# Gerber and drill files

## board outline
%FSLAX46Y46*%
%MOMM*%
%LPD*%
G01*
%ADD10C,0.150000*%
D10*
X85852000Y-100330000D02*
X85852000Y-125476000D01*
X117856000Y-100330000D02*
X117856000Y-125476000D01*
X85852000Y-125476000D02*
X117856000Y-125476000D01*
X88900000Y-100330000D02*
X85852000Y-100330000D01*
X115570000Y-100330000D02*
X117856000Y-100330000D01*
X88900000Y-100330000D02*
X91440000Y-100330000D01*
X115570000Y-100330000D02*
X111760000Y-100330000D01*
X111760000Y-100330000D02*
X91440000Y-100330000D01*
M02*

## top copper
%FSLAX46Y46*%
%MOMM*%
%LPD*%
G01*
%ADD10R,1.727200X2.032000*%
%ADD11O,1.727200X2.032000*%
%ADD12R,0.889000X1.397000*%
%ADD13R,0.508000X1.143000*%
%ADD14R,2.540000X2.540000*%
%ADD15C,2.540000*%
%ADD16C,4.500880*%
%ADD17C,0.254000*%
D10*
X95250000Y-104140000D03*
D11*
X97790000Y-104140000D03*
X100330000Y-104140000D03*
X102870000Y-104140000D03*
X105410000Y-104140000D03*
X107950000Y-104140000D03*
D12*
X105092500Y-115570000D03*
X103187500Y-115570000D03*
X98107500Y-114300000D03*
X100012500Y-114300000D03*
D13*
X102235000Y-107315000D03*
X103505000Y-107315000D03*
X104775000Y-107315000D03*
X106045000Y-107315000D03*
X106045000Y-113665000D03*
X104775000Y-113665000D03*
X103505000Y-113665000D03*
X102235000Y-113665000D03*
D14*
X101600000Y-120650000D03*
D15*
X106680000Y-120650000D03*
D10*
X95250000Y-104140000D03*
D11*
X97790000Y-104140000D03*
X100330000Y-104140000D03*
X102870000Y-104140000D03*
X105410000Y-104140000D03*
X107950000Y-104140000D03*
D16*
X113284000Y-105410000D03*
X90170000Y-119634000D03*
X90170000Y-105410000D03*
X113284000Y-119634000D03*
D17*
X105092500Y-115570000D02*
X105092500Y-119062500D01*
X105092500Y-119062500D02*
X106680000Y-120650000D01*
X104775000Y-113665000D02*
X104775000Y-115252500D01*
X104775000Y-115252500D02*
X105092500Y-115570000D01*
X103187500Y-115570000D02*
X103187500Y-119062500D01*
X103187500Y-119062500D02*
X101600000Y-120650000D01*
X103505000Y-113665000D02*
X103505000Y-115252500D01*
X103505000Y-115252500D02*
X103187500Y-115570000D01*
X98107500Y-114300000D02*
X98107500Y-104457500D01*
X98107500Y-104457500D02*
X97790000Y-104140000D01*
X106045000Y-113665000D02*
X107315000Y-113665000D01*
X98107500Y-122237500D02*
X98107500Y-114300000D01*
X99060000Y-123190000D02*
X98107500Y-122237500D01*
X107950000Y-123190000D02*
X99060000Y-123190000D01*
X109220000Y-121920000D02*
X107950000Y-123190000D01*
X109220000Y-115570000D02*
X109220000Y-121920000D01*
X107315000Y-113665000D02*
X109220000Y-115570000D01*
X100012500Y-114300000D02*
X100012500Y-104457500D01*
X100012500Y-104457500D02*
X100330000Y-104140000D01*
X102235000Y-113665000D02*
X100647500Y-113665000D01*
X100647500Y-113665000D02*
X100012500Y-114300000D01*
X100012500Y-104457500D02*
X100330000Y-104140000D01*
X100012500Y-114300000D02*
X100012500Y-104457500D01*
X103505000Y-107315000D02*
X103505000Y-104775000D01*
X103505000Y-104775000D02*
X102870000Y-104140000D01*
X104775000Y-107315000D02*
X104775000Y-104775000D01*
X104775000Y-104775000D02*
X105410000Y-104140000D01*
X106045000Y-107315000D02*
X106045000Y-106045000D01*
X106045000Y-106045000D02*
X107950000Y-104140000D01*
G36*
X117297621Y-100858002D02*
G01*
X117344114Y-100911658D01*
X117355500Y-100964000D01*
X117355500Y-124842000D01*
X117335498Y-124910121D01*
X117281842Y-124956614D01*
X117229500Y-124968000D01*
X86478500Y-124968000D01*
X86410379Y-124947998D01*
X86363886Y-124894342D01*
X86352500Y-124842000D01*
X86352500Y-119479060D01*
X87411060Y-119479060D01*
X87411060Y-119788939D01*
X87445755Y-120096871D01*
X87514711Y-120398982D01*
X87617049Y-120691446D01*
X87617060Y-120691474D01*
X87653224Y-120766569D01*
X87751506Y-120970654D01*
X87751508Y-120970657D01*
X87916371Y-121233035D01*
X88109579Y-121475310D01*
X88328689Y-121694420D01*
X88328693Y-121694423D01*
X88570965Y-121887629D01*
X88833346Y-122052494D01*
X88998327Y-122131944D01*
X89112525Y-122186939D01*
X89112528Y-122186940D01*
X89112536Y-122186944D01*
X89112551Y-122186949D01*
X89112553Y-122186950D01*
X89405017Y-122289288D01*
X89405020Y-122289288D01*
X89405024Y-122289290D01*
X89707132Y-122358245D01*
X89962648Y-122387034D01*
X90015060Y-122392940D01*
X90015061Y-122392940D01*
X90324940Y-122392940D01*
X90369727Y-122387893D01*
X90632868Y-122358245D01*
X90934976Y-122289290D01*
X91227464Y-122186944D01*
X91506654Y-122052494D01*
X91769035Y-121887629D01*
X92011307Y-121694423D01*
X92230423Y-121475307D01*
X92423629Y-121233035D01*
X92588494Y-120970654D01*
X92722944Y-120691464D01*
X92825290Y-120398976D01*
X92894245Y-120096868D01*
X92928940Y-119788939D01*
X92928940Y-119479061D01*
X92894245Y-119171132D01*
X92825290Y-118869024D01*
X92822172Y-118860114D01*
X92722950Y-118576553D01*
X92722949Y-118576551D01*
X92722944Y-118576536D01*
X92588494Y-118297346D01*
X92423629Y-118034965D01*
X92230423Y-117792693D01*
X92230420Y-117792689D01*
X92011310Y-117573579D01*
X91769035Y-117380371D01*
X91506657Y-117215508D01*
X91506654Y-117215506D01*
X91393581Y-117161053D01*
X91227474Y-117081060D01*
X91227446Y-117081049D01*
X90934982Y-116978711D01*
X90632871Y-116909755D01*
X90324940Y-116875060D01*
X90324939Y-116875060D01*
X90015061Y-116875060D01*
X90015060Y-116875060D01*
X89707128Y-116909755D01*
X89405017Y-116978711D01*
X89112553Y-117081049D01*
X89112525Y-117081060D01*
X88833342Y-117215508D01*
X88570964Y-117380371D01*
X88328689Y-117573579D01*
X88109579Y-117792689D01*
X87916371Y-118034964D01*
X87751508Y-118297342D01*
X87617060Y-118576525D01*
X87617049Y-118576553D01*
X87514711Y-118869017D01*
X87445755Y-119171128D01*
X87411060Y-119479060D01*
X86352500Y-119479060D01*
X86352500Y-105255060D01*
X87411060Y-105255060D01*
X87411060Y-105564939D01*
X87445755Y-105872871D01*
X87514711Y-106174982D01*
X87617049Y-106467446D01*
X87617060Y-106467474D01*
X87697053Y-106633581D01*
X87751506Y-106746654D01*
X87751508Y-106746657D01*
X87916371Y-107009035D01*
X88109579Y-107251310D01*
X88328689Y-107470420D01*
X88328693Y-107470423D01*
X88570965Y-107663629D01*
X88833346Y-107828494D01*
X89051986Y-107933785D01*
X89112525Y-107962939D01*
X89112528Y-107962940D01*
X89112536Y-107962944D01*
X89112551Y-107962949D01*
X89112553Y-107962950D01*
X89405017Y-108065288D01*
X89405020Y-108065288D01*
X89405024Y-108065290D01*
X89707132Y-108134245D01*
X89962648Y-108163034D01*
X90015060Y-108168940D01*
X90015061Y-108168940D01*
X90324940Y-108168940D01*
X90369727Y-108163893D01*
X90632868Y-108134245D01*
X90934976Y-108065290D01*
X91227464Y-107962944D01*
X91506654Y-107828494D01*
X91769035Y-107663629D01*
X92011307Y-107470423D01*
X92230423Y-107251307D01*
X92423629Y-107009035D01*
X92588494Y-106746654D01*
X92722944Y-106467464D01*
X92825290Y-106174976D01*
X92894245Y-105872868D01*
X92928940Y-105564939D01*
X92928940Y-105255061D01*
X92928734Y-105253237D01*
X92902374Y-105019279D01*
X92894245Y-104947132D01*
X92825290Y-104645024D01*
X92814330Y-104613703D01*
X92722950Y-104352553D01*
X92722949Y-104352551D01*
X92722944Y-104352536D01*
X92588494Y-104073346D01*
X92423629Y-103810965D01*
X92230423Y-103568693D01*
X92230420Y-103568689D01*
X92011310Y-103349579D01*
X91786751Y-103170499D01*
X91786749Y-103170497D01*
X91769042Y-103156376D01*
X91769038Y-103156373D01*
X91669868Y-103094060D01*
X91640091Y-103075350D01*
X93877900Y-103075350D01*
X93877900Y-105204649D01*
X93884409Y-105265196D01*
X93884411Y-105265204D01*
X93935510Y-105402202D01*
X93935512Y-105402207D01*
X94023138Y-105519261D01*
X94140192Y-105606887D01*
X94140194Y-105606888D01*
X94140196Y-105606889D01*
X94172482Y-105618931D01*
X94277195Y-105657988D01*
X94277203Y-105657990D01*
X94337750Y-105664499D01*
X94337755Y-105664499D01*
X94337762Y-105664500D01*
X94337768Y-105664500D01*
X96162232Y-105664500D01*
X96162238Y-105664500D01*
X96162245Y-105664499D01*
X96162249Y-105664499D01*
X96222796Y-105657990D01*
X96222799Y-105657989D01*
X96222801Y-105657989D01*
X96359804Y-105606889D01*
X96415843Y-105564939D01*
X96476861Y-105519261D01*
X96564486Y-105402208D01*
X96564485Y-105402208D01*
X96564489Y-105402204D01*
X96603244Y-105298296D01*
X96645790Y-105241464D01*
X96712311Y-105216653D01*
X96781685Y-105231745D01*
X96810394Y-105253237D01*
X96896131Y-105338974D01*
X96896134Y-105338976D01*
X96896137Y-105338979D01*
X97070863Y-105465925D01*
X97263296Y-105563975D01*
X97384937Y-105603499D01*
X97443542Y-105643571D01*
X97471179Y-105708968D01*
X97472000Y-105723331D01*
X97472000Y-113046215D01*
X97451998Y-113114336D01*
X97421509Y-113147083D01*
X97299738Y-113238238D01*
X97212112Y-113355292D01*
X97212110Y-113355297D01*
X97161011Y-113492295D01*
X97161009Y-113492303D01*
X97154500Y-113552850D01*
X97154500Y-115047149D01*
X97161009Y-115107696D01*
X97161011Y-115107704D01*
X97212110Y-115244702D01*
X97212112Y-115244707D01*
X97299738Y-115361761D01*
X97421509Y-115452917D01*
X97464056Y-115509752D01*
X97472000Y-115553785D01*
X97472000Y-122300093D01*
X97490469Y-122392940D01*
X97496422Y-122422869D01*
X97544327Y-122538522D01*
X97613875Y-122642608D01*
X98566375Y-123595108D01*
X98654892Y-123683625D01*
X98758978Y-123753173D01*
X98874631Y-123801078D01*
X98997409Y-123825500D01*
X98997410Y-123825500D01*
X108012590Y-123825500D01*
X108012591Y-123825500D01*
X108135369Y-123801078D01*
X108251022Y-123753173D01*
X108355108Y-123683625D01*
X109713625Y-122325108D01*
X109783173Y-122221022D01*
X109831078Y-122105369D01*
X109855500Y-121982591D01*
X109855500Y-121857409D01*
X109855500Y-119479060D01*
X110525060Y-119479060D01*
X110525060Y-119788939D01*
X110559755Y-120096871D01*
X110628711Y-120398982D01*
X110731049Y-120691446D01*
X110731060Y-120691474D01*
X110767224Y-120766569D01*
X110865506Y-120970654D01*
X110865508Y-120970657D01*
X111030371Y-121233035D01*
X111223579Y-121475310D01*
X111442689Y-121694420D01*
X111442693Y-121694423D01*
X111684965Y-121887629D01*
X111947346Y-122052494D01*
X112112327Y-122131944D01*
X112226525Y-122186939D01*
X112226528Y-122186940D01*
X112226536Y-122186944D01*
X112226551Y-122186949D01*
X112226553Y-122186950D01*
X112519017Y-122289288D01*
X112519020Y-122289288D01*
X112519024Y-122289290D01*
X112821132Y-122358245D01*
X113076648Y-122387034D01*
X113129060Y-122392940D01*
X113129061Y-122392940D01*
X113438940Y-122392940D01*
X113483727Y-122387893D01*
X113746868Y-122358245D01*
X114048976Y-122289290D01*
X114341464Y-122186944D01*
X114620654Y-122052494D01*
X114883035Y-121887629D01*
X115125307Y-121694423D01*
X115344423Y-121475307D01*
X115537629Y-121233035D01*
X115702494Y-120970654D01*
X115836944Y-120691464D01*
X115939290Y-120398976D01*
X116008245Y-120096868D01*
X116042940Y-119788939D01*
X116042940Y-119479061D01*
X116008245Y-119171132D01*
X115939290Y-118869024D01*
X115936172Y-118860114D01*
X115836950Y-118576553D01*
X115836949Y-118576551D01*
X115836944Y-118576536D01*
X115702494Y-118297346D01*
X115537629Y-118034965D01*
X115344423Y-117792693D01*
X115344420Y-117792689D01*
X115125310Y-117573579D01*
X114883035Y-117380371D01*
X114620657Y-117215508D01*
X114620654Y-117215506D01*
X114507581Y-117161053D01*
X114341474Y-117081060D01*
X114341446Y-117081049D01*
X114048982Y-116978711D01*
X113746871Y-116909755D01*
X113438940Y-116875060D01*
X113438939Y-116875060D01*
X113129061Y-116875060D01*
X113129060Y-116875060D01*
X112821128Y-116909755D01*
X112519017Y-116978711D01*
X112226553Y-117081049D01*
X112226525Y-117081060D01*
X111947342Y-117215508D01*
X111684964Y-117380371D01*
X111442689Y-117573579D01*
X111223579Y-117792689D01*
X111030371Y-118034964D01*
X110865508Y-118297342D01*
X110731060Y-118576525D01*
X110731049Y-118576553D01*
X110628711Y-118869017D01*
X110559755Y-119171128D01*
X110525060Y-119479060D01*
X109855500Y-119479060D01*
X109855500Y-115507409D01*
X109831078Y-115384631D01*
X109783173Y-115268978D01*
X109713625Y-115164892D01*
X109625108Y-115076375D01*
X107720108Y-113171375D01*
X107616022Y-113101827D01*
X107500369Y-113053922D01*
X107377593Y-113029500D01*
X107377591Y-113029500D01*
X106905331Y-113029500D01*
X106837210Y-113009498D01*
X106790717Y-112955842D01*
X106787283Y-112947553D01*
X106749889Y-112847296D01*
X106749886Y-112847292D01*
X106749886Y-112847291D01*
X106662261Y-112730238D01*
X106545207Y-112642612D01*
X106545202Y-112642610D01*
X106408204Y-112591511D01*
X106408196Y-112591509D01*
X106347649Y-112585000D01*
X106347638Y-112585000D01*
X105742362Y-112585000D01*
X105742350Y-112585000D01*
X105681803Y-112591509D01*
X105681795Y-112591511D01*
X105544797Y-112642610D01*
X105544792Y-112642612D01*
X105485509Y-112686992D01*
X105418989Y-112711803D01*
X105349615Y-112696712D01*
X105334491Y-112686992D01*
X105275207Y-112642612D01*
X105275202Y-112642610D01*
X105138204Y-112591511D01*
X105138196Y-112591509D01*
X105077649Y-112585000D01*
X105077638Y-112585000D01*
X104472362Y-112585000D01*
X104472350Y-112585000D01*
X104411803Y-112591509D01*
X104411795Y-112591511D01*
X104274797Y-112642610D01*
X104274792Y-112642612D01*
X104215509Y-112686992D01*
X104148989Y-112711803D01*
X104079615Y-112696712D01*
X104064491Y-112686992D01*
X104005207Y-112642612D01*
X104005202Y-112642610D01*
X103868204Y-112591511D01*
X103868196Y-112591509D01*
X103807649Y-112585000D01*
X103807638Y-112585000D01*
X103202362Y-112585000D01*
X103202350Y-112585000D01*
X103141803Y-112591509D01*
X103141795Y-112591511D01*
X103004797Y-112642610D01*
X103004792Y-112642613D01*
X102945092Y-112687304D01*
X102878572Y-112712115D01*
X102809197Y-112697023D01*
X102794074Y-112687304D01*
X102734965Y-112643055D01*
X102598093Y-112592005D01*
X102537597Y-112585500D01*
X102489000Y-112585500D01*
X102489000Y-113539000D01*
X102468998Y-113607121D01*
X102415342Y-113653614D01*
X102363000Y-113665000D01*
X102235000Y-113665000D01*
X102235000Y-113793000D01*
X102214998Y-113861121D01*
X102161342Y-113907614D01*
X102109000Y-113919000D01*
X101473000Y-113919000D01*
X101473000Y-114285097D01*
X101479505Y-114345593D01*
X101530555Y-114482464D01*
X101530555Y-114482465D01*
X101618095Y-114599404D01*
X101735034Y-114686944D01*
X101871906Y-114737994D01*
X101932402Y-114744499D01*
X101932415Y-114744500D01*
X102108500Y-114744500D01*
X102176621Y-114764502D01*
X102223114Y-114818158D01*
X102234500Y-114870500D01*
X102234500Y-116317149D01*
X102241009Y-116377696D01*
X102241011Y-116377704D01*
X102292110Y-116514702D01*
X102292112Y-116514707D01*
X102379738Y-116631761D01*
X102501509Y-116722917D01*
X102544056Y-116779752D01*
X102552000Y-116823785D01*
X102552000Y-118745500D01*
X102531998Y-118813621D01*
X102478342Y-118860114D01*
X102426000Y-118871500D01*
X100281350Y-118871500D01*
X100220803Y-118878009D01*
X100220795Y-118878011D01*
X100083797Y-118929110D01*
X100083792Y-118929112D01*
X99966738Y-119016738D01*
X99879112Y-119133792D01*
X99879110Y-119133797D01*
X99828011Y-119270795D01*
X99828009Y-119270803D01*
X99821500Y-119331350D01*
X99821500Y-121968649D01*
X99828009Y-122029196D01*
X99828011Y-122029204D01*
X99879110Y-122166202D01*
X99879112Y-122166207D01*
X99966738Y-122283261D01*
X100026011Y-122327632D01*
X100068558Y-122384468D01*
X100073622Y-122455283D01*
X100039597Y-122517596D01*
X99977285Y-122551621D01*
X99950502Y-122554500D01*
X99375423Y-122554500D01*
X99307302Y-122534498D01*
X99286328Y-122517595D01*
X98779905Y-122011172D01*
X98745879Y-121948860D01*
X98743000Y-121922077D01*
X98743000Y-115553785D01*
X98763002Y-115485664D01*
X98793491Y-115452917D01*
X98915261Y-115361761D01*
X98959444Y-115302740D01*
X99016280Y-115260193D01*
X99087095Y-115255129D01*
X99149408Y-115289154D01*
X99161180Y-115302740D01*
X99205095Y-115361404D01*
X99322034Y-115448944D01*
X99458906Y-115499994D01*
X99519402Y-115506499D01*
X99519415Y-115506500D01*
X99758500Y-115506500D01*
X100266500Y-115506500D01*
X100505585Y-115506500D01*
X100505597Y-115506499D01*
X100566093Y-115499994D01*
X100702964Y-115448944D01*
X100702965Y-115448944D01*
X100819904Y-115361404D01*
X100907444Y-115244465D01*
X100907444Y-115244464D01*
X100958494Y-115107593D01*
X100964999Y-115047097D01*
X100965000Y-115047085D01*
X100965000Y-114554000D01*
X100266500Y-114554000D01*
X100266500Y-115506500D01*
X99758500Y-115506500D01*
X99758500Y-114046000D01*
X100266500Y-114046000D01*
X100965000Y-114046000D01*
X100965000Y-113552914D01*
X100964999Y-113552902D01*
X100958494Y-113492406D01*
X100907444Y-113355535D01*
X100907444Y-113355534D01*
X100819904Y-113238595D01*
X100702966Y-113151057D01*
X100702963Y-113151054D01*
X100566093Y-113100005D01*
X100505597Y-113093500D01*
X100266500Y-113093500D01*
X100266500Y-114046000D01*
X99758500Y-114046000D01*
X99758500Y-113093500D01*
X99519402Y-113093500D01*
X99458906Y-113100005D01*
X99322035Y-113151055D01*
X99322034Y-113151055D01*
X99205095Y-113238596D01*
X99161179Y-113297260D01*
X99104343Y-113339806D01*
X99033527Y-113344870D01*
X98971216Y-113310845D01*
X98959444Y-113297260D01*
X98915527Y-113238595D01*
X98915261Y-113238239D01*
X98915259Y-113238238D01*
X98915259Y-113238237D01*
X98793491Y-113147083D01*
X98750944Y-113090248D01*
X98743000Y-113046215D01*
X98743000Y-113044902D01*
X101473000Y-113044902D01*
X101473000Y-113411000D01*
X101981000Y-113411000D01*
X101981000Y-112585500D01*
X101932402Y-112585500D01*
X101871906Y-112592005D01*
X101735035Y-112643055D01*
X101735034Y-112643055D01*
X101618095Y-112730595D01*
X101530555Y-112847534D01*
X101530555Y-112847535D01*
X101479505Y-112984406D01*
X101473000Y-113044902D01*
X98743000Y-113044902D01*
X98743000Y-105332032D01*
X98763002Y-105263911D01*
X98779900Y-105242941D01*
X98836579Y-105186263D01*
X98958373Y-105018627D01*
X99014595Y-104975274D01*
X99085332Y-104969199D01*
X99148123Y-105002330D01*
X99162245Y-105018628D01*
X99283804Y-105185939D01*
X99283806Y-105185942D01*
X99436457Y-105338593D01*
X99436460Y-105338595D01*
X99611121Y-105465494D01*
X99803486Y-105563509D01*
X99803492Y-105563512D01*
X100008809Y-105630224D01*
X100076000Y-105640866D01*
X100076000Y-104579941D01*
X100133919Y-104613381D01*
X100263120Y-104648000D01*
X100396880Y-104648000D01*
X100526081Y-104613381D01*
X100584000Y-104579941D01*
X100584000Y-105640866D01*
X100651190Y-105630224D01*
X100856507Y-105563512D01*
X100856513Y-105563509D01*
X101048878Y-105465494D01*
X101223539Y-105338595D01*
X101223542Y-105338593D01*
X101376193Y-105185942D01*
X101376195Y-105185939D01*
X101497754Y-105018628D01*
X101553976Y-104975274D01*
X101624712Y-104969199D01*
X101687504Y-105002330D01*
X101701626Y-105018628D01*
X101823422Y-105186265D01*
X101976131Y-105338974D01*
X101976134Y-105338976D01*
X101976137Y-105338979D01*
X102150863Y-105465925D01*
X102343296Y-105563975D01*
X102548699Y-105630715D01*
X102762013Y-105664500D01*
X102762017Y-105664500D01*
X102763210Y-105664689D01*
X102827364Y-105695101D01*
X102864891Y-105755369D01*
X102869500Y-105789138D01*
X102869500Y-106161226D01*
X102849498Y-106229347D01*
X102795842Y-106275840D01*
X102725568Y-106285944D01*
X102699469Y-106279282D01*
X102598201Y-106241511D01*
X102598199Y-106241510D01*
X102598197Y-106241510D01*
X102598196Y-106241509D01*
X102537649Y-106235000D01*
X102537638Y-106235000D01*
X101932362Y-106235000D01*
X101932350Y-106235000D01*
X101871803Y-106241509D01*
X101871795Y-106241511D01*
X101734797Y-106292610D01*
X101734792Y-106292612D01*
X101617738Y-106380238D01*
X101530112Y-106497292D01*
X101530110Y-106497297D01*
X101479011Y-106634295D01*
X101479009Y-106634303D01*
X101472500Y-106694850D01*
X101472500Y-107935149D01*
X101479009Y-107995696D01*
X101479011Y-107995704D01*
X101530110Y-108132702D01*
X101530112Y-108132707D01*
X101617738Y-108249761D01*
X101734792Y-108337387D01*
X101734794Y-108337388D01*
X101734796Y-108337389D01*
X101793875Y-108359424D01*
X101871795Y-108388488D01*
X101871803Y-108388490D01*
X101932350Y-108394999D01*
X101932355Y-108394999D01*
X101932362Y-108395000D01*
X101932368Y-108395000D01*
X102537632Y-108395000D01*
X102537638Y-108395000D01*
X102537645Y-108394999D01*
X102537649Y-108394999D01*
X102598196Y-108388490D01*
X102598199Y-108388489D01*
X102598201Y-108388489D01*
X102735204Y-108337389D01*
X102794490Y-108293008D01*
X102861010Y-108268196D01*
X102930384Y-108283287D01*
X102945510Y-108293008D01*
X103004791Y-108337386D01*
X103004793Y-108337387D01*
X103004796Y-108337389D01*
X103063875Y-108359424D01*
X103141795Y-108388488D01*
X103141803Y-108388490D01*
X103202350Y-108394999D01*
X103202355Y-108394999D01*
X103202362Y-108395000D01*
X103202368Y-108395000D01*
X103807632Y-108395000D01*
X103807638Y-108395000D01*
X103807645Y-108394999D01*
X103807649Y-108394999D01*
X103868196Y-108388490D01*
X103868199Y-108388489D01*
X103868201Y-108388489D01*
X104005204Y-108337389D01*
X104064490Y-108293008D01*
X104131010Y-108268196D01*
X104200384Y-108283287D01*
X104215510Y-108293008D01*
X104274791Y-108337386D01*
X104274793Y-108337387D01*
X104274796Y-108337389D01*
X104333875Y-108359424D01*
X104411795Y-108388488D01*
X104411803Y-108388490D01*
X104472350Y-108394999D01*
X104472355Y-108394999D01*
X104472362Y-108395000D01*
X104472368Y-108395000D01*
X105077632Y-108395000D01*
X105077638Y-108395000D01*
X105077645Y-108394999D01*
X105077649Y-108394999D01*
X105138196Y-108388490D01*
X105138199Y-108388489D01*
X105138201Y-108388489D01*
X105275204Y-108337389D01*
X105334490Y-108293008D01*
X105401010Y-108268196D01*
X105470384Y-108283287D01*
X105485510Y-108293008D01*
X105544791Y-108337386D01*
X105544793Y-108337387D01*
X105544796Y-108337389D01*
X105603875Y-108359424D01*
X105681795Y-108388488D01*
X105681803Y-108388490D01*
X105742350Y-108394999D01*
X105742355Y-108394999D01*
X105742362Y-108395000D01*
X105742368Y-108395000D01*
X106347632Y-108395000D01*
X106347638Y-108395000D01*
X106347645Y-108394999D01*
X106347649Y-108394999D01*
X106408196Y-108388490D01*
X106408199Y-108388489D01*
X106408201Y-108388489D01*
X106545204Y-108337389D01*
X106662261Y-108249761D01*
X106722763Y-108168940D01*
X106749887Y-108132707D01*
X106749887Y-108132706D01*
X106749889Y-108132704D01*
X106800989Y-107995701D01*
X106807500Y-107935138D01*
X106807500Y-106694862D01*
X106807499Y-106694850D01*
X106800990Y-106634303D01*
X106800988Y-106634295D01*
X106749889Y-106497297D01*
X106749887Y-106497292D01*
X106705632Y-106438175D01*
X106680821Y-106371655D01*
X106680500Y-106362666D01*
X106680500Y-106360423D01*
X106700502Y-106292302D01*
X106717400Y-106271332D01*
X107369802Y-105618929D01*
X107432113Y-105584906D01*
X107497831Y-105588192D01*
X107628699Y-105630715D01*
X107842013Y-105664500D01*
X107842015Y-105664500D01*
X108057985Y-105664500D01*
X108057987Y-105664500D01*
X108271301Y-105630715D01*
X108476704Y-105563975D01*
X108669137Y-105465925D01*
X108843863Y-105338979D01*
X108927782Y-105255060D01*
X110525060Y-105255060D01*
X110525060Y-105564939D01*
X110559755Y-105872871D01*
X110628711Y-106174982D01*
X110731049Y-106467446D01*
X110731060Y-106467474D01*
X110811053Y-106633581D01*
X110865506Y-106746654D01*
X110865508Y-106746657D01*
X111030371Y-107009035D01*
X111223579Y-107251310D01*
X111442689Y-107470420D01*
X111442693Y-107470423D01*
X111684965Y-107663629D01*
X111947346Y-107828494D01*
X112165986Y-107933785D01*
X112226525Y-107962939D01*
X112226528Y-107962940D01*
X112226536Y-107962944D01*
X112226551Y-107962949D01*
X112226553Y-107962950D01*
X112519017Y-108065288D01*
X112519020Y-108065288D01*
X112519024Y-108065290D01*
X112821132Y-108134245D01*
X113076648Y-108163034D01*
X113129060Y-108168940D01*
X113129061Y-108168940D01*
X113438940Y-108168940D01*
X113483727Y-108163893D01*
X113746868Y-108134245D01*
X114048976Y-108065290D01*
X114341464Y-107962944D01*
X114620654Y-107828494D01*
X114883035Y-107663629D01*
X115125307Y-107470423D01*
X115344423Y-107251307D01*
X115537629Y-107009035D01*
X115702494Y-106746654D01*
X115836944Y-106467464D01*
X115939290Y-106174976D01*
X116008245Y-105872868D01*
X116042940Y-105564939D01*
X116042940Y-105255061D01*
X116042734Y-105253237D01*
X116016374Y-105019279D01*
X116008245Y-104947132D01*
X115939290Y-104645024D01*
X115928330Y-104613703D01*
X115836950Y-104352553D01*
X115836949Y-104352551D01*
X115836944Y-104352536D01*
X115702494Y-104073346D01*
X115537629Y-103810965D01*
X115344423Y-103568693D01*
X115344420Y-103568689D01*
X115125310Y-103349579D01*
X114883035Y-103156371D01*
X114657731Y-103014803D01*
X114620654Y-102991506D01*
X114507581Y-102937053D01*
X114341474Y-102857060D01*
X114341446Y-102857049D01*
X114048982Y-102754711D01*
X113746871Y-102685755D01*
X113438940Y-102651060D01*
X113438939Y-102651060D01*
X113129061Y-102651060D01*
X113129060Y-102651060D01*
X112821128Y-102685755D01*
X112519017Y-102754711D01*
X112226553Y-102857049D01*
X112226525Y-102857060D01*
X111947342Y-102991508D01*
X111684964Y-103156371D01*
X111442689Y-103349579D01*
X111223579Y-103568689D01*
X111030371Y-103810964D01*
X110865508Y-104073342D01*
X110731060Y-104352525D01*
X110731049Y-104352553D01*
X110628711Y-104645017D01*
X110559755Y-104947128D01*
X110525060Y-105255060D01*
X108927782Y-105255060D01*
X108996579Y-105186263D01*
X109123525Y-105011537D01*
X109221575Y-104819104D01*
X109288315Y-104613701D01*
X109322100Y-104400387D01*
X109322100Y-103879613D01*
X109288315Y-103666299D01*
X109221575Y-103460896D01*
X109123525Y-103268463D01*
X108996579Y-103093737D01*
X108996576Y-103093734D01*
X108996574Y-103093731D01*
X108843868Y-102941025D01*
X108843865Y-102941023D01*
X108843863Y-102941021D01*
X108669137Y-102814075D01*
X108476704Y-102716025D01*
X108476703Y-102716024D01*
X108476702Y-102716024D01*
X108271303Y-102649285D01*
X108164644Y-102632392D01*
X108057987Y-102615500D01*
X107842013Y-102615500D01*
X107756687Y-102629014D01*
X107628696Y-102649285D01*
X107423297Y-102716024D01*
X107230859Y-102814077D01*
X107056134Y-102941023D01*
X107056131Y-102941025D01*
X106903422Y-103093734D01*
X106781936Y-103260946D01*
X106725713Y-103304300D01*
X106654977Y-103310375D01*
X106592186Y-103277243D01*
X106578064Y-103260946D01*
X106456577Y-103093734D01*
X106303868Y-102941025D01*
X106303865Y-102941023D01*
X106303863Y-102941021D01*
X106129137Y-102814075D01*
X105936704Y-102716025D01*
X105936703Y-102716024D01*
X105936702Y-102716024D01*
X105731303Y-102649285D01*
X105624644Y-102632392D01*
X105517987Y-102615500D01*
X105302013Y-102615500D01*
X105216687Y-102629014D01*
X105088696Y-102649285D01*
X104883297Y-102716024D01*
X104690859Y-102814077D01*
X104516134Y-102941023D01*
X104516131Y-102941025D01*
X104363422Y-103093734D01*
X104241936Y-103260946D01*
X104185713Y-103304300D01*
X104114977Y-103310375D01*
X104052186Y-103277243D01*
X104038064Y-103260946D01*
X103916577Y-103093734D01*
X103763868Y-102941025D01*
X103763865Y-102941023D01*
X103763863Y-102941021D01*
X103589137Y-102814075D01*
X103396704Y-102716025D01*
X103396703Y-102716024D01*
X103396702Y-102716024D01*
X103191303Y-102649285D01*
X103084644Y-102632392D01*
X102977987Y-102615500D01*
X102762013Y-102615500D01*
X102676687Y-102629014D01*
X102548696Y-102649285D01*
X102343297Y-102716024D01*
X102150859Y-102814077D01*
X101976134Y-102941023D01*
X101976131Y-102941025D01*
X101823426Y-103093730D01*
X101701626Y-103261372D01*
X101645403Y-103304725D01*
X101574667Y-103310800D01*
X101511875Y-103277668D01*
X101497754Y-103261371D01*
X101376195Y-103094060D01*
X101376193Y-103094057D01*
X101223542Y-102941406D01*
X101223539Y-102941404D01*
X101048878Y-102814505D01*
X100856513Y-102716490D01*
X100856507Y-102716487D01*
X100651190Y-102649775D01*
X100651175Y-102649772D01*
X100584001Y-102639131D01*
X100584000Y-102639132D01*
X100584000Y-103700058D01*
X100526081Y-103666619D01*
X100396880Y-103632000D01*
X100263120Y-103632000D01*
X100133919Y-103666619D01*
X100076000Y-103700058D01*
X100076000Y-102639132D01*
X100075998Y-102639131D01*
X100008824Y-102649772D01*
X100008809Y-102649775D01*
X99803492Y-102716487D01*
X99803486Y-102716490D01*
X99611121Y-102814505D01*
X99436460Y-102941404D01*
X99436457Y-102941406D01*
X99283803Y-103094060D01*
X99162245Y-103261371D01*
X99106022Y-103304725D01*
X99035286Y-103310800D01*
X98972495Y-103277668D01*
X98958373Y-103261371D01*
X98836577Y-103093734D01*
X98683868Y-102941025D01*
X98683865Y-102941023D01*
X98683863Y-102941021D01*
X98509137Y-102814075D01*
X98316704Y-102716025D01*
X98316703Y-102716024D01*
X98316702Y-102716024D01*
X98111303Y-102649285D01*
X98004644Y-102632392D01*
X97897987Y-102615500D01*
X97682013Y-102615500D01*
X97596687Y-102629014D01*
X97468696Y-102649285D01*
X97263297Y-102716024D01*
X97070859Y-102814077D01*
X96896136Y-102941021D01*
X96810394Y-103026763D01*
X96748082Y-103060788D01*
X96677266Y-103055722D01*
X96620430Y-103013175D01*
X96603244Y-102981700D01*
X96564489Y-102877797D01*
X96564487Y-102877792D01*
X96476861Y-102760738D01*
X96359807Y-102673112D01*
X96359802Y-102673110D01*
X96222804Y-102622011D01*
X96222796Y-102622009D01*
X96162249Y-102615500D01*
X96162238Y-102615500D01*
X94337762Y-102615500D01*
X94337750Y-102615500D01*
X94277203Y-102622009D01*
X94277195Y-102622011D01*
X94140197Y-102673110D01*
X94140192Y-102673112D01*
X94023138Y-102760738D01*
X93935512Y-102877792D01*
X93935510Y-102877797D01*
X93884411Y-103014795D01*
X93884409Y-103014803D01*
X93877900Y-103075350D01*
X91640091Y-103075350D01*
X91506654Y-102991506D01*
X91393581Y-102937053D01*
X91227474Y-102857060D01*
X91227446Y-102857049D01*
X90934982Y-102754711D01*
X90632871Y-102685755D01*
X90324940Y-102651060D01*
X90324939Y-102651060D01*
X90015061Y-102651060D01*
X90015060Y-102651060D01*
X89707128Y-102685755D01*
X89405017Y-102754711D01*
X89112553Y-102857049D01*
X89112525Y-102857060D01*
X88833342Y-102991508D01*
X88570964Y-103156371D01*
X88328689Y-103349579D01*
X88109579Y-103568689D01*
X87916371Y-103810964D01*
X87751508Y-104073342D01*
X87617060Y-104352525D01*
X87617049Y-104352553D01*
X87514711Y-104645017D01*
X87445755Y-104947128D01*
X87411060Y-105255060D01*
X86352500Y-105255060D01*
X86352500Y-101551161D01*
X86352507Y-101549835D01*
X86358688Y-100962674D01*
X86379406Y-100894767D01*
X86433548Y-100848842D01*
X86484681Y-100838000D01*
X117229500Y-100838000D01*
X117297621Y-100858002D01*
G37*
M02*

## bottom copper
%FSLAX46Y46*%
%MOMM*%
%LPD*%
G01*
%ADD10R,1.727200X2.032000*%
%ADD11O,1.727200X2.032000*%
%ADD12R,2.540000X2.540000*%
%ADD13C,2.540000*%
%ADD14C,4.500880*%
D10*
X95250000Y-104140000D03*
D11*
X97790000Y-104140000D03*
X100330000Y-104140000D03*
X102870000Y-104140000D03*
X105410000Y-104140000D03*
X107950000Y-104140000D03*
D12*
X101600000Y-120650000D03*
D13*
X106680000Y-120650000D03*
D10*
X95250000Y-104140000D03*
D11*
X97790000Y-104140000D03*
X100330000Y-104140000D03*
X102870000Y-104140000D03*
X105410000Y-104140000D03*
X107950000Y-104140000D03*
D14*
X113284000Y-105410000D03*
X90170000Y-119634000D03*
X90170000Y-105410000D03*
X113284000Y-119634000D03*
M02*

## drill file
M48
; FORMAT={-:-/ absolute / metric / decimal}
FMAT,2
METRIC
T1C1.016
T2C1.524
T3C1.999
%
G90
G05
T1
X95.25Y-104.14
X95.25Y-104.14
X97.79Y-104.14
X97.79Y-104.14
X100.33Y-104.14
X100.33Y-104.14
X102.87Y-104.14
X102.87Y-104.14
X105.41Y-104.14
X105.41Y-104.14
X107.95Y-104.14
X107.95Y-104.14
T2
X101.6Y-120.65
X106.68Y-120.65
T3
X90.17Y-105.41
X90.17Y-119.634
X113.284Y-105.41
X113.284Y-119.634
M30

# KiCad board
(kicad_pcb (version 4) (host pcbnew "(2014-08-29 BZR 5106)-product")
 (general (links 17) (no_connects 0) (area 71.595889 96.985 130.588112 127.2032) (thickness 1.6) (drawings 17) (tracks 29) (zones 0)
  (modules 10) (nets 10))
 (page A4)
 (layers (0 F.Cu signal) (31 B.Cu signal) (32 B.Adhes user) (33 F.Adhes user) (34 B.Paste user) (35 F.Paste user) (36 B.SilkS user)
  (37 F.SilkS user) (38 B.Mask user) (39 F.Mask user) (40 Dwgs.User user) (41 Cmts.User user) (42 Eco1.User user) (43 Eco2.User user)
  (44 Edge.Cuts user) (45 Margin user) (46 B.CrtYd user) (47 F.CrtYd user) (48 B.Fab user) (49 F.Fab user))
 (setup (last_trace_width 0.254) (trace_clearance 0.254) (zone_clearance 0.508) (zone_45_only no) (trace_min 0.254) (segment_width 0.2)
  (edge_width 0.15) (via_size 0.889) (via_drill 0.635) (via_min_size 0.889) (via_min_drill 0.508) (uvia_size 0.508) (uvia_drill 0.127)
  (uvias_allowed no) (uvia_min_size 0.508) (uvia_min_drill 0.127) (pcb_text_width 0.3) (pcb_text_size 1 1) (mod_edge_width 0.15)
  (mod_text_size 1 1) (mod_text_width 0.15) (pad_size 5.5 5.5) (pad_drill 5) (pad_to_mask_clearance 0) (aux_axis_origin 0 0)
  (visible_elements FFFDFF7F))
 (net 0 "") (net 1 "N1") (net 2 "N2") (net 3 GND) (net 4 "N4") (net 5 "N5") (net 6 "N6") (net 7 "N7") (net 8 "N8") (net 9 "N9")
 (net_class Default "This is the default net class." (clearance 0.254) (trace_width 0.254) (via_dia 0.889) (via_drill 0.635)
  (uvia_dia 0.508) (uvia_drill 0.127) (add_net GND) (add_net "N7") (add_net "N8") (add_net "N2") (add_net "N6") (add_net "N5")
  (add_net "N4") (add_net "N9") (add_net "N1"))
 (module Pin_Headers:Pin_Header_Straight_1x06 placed (layer F.Cu) (at 101.6 104.14)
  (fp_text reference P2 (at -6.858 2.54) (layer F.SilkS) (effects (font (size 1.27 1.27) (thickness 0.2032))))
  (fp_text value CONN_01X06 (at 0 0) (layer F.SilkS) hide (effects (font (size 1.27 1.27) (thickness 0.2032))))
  (pad 1 thru_hole rect (at -6.35 0) (size 1.7272 2.032) (drill 1.016) (layers *.Cu *.Mask F.SilkS) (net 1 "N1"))
  (pad 2 thru_hole oval (at -3.81 0) (size 1.7272 2.032) (drill 1.016) (layers *.Cu *.Mask F.SilkS) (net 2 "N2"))
  (pad 3 thru_hole oval (at -1.27 0) (size 1.7272 2.032) (drill 1.016) (layers *.Cu *.Mask F.SilkS) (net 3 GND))
  (pad 4 thru_hole oval (at 1.27 0) (size 1.7272 2.032) (drill 1.016) (layers *.Cu *.Mask F.SilkS) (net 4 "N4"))
  (pad 5 thru_hole oval (at 3.81 0) (size 1.7272 2.032) (drill 1.016) (layers *.Cu *.Mask F.SilkS) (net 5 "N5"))
  (pad 6 thru_hole oval (at 6.35 0) (size 1.7272 2.032) (drill 1.016) (layers *.Cu *.Mask F.SilkS) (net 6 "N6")))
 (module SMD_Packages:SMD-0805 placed (layer F.Cu) (at 104.14 115.57 180)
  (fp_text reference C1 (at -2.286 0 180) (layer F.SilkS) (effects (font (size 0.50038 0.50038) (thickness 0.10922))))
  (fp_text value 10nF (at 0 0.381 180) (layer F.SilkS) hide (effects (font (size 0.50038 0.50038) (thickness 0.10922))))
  (pad 1 smd rect (at -0.9525 0 180) (size 0.889 1.397) (layers F.Cu F.Paste F.Mask) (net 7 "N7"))
  (pad 2 smd rect (at 0.9525 0 180) (size 0.889 1.397) (layers F.Cu F.Paste F.Mask) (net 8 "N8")))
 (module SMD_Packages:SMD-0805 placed (layer F.Cu) (at 99.06 114.3)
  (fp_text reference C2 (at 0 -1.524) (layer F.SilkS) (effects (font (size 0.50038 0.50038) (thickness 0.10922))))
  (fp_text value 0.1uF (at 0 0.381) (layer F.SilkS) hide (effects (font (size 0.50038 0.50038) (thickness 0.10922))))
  (pad 1 smd rect (at -0.9525 0) (size 0.889 1.397) (layers F.Cu F.Paste F.Mask) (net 2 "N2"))
  (pad 2 smd rect (at 0.9525 0) (size 0.889 1.397) (layers F.Cu F.Paste F.Mask) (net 3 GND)))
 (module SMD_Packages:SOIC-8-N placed (layer F.Cu) (at 104.14 110.49)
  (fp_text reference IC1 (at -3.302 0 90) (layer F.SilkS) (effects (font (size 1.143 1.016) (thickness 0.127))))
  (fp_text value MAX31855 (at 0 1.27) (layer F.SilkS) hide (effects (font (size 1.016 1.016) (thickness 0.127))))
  (pad 8 smd rect (at -1.905 -3.175) (size 0.508 1.143) (layers F.Cu F.Paste F.Mask) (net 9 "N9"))
  (pad 7 smd rect (at -0.635 -3.175) (size 0.508 1.143) (layers F.Cu F.Paste F.Mask) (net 4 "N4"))
  (pad 6 smd rect (at 0.635 -3.175) (size 0.508 1.143) (layers F.Cu F.Paste F.Mask) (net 5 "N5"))
  (pad 5 smd rect (at 1.905 -3.175) (size 0.508 1.143) (layers F.Cu F.Paste F.Mask) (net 6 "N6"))
  (pad 4 smd rect (at 1.905 3.175) (size 0.508 1.143) (layers F.Cu F.Paste F.Mask) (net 2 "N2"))
  (pad 3 smd rect (at 0.635 3.175) (size 0.508 1.143) (layers F.Cu F.Paste F.Mask) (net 7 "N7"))
  (pad 2 smd rect (at -0.635 3.175) (size 0.508 1.143) (layers F.Cu F.Paste F.Mask) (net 8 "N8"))
  (pad 1 smd rect (at -1.905 3.175) (size 0.508 1.143) (layers F.Cu F.Paste F.Mask) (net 3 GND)))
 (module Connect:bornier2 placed (layer F.Cu) (at 104.14 120.65)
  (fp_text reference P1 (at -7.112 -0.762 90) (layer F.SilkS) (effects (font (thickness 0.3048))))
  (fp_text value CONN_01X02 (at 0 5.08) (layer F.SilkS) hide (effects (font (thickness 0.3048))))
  (pad 1 thru_hole rect (at -2.54 0) (size 2.54 2.54) (drill 1.524) (layers *.Cu *.Mask F.SilkS) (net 8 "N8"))
  (pad 2 thru_hole circle (at 2.54 0) (size 2.54 2.54) (drill 1.524) (layers *.Cu *.Mask F.SilkS) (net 7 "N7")))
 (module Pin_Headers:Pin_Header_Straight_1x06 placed (layer F.Cu) (at 101.6 104.14)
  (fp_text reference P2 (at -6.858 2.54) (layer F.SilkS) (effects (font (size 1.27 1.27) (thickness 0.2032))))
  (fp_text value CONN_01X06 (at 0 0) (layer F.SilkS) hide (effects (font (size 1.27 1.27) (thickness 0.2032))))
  (pad 1 thru_hole rect (at -6.35 0) (size 1.7272 2.032) (drill 1.016) (layers *.Cu *.Mask F.SilkS) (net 1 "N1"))
  (pad 2 thru_hole oval (at -3.81 0) (size 1.7272 2.032) (drill 1.016) (layers *.Cu *.Mask F.SilkS) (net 2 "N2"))
  (pad 3 thru_hole oval (at -1.27 0) (size 1.7272 2.032) (drill 1.016) (layers *.Cu *.Mask F.SilkS) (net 3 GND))
  (pad 4 thru_hole oval (at 1.27 0) (size 1.7272 2.032) (drill 1.016) (layers *.Cu *.Mask F.SilkS) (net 4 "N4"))
  (pad 5 thru_hole oval (at 3.81 0) (size 1.7272 2.032) (drill 1.016) (layers *.Cu *.Mask F.SilkS) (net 5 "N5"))
  (pad 6 thru_hole oval (at 6.35 0) (size 1.7272 2.032) (drill 1.016) (layers *.Cu *.Mask F.SilkS) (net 6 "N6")))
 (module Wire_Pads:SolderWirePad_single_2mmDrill (layer F.Cu) (at 113.284 105.41)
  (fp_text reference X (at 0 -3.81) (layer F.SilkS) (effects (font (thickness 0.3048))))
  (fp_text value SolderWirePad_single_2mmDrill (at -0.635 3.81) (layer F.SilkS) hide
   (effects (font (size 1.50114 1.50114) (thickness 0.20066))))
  (pad 1 thru_hole circle (at 0 0) (size 4.50088 4.50088) (drill 1.99898) (layers *.Cu *.Mask F.SilkS)))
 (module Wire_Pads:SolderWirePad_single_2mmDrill (layer F.Cu) (at 90.17 119.634)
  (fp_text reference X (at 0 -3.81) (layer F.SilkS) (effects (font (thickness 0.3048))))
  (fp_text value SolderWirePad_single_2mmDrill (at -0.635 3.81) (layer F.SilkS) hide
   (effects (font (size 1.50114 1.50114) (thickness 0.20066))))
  (pad 1 thru_hole circle (at 0 0) (size 4.50088 4.50088) (drill 1.99898) (layers *.Cu *.Mask F.SilkS)))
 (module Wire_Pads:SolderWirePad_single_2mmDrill (layer F.Cu) (at 90.17 105.41)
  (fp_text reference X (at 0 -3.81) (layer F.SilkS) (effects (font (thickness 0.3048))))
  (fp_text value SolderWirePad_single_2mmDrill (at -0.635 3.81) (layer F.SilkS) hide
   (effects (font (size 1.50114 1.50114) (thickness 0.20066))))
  (pad 1 thru_hole circle (at 0 0) (size 4.50088 4.50088) (drill 1.99898) (layers *.Cu *.Mask F.SilkS)))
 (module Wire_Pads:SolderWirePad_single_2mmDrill (layer F.Cu) (at 113.284 119.634)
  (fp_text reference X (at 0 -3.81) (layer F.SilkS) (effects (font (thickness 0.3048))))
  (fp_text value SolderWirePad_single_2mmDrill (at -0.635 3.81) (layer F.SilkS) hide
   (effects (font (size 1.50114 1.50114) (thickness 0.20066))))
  (pad 1 thru_hole circle (at 0 0) (size 4.50088 4.50088) (drill 1.99898) (layers *.Cu *.Mask F.SilkS)))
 (gr_line (start 85.852 100.33) (end 85.852 125.476) (angle 90) (layer Edge.Cuts) (width 0.15))
 (gr_line (start 117.856 100.33) (end 117.856 125.476) (angle 90) (layer Edge.Cuts) (width 0.15))
 (gr_line (start 85.852 125.476) (end 117.856 125.476) (angle 90) (layer Edge.Cuts) (width 0.15))
 (gr_line (start 88.9 100.33) (end 85.852 100.33) (angle 90) (layer Edge.Cuts) (width 0.15))
 (gr_line (start 115.57 100.33) (end 117.856 100.33) (angle 90) (layer Edge.Cuts) (width 0.15))
 (gr_line (start 88.9 100.33) (end 91.44 100.33) (angle 90) (layer Edge.Cuts) (width 0.15))
 (gr_line (start 115.57 100.33) (end 111.76 100.33) (angle 90) (layer Edge.Cuts) (width 0.15))
 (gr_line (start 111.76 100.33) (end 91.44 100.33) (angle 90) (layer Edge.Cuts) (width 0.15))
 (segment (start 105.0925 115.57) (end 105.0925 119.0625) (width 0.254) (layer F.Cu) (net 7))
 (segment (start 105.0925 119.0625) (end 106.68 120.65) (width 0.254) (layer F.Cu) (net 7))
 (segment (start 104.775 113.665) (end 104.775 115.2525) (width 0.254) (layer F.Cu) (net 7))
 (segment (start 104.775 115.2525) (end 105.0925 115.57) (width 0.254) (layer F.Cu) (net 7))
 (segment (start 103.1875 115.57) (end 103.1875 119.0625) (width 0.254) (layer F.Cu) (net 8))
 (segment (start 103.1875 119.0625) (end 101.6 120.65) (width 0.254) (layer F.Cu) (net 8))
 (segment (start 103.505 113.665) (end 103.505 115.2525) (width 0.254) (layer F.Cu) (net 8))
 (segment (start 103.505 115.2525) (end 103.1875 115.57) (width 0.254) (layer F.Cu) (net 8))
 (segment (start 98.1075 114.3) (end 98.1075 104.4575) (width 0.254) (layer F.Cu) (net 2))
 (segment (start 98.1075 104.4575) (end 97.79 104.14) (width 0.254) (layer F.Cu) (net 2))
 (segment (start 106.045 113.665) (end 107.315 113.665) (width 0.254) (layer F.Cu) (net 2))
 (segment (start 98.1075 122.2375) (end 98.1075 114.3) (width 0.254) (layer F.Cu) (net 2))
 (segment (start 99.06 123.19) (end 98.1075 122.2375) (width 0.254) (layer F.Cu) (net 2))
 (segment (start 107.95 123.19) (end 99.06 123.19) (width 0.254) (layer F.Cu) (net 2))
 (segment (start 109.22 121.92) (end 107.95 123.19) (width 0.254) (layer F.Cu) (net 2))
 (segment (start 109.22 115.57) (end 109.22 121.92) (width 0.254) (layer F.Cu) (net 2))
 (segment (start 107.315 113.665) (end 109.22 115.57) (width 0.254) (layer F.Cu) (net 2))
 (segment (start 100.0125 114.3) (end 100.0125 104.4575) (width 0.254) (layer F.Cu) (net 3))
 (segment (start 100.0125 104.4575) (end 100.33 104.14) (width 0.254) (layer F.Cu) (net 3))
 (segment (start 102.235 113.665) (end 100.6475 113.665) (width 0.254) (layer F.Cu) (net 3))
 (segment (start 100.6475 113.665) (end 100.0125 114.3) (width 0.254) (layer F.Cu) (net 3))
 (segment (start 100.0125 104.4575) (end 100.33 104.14) (width 0.254) (layer F.Cu) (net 3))
 (segment (start 100.0125 114.3) (end 100.0125 104.4575) (width 0.254) (layer F.Cu) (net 3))
 (segment (start 103.505 107.315) (end 103.505 104.775) (width 0.254) (layer F.Cu) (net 4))
 (segment (start 103.505 104.775) (end 102.87 104.14) (width 0.254) (layer F.Cu) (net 4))
 (segment (start 104.775 107.315) (end 104.775 104.775) (width 0.254) (layer F.Cu) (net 5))
 (segment (start 104.775 104.775) (end 105.41 104.14) (width 0.254) (layer F.Cu) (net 5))
 (segment (start 106.045 107.315) (end 106.045 106.045) (width 0.254) (layer F.Cu) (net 6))
 (segment (start 106.045 106.045) (end 107.95 104.14) (width 0.254) (layer F.Cu) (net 6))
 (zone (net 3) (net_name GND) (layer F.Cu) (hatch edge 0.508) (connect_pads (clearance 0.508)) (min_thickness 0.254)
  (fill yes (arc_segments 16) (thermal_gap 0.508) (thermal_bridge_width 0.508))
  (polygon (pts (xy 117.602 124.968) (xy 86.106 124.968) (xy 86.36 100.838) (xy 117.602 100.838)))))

